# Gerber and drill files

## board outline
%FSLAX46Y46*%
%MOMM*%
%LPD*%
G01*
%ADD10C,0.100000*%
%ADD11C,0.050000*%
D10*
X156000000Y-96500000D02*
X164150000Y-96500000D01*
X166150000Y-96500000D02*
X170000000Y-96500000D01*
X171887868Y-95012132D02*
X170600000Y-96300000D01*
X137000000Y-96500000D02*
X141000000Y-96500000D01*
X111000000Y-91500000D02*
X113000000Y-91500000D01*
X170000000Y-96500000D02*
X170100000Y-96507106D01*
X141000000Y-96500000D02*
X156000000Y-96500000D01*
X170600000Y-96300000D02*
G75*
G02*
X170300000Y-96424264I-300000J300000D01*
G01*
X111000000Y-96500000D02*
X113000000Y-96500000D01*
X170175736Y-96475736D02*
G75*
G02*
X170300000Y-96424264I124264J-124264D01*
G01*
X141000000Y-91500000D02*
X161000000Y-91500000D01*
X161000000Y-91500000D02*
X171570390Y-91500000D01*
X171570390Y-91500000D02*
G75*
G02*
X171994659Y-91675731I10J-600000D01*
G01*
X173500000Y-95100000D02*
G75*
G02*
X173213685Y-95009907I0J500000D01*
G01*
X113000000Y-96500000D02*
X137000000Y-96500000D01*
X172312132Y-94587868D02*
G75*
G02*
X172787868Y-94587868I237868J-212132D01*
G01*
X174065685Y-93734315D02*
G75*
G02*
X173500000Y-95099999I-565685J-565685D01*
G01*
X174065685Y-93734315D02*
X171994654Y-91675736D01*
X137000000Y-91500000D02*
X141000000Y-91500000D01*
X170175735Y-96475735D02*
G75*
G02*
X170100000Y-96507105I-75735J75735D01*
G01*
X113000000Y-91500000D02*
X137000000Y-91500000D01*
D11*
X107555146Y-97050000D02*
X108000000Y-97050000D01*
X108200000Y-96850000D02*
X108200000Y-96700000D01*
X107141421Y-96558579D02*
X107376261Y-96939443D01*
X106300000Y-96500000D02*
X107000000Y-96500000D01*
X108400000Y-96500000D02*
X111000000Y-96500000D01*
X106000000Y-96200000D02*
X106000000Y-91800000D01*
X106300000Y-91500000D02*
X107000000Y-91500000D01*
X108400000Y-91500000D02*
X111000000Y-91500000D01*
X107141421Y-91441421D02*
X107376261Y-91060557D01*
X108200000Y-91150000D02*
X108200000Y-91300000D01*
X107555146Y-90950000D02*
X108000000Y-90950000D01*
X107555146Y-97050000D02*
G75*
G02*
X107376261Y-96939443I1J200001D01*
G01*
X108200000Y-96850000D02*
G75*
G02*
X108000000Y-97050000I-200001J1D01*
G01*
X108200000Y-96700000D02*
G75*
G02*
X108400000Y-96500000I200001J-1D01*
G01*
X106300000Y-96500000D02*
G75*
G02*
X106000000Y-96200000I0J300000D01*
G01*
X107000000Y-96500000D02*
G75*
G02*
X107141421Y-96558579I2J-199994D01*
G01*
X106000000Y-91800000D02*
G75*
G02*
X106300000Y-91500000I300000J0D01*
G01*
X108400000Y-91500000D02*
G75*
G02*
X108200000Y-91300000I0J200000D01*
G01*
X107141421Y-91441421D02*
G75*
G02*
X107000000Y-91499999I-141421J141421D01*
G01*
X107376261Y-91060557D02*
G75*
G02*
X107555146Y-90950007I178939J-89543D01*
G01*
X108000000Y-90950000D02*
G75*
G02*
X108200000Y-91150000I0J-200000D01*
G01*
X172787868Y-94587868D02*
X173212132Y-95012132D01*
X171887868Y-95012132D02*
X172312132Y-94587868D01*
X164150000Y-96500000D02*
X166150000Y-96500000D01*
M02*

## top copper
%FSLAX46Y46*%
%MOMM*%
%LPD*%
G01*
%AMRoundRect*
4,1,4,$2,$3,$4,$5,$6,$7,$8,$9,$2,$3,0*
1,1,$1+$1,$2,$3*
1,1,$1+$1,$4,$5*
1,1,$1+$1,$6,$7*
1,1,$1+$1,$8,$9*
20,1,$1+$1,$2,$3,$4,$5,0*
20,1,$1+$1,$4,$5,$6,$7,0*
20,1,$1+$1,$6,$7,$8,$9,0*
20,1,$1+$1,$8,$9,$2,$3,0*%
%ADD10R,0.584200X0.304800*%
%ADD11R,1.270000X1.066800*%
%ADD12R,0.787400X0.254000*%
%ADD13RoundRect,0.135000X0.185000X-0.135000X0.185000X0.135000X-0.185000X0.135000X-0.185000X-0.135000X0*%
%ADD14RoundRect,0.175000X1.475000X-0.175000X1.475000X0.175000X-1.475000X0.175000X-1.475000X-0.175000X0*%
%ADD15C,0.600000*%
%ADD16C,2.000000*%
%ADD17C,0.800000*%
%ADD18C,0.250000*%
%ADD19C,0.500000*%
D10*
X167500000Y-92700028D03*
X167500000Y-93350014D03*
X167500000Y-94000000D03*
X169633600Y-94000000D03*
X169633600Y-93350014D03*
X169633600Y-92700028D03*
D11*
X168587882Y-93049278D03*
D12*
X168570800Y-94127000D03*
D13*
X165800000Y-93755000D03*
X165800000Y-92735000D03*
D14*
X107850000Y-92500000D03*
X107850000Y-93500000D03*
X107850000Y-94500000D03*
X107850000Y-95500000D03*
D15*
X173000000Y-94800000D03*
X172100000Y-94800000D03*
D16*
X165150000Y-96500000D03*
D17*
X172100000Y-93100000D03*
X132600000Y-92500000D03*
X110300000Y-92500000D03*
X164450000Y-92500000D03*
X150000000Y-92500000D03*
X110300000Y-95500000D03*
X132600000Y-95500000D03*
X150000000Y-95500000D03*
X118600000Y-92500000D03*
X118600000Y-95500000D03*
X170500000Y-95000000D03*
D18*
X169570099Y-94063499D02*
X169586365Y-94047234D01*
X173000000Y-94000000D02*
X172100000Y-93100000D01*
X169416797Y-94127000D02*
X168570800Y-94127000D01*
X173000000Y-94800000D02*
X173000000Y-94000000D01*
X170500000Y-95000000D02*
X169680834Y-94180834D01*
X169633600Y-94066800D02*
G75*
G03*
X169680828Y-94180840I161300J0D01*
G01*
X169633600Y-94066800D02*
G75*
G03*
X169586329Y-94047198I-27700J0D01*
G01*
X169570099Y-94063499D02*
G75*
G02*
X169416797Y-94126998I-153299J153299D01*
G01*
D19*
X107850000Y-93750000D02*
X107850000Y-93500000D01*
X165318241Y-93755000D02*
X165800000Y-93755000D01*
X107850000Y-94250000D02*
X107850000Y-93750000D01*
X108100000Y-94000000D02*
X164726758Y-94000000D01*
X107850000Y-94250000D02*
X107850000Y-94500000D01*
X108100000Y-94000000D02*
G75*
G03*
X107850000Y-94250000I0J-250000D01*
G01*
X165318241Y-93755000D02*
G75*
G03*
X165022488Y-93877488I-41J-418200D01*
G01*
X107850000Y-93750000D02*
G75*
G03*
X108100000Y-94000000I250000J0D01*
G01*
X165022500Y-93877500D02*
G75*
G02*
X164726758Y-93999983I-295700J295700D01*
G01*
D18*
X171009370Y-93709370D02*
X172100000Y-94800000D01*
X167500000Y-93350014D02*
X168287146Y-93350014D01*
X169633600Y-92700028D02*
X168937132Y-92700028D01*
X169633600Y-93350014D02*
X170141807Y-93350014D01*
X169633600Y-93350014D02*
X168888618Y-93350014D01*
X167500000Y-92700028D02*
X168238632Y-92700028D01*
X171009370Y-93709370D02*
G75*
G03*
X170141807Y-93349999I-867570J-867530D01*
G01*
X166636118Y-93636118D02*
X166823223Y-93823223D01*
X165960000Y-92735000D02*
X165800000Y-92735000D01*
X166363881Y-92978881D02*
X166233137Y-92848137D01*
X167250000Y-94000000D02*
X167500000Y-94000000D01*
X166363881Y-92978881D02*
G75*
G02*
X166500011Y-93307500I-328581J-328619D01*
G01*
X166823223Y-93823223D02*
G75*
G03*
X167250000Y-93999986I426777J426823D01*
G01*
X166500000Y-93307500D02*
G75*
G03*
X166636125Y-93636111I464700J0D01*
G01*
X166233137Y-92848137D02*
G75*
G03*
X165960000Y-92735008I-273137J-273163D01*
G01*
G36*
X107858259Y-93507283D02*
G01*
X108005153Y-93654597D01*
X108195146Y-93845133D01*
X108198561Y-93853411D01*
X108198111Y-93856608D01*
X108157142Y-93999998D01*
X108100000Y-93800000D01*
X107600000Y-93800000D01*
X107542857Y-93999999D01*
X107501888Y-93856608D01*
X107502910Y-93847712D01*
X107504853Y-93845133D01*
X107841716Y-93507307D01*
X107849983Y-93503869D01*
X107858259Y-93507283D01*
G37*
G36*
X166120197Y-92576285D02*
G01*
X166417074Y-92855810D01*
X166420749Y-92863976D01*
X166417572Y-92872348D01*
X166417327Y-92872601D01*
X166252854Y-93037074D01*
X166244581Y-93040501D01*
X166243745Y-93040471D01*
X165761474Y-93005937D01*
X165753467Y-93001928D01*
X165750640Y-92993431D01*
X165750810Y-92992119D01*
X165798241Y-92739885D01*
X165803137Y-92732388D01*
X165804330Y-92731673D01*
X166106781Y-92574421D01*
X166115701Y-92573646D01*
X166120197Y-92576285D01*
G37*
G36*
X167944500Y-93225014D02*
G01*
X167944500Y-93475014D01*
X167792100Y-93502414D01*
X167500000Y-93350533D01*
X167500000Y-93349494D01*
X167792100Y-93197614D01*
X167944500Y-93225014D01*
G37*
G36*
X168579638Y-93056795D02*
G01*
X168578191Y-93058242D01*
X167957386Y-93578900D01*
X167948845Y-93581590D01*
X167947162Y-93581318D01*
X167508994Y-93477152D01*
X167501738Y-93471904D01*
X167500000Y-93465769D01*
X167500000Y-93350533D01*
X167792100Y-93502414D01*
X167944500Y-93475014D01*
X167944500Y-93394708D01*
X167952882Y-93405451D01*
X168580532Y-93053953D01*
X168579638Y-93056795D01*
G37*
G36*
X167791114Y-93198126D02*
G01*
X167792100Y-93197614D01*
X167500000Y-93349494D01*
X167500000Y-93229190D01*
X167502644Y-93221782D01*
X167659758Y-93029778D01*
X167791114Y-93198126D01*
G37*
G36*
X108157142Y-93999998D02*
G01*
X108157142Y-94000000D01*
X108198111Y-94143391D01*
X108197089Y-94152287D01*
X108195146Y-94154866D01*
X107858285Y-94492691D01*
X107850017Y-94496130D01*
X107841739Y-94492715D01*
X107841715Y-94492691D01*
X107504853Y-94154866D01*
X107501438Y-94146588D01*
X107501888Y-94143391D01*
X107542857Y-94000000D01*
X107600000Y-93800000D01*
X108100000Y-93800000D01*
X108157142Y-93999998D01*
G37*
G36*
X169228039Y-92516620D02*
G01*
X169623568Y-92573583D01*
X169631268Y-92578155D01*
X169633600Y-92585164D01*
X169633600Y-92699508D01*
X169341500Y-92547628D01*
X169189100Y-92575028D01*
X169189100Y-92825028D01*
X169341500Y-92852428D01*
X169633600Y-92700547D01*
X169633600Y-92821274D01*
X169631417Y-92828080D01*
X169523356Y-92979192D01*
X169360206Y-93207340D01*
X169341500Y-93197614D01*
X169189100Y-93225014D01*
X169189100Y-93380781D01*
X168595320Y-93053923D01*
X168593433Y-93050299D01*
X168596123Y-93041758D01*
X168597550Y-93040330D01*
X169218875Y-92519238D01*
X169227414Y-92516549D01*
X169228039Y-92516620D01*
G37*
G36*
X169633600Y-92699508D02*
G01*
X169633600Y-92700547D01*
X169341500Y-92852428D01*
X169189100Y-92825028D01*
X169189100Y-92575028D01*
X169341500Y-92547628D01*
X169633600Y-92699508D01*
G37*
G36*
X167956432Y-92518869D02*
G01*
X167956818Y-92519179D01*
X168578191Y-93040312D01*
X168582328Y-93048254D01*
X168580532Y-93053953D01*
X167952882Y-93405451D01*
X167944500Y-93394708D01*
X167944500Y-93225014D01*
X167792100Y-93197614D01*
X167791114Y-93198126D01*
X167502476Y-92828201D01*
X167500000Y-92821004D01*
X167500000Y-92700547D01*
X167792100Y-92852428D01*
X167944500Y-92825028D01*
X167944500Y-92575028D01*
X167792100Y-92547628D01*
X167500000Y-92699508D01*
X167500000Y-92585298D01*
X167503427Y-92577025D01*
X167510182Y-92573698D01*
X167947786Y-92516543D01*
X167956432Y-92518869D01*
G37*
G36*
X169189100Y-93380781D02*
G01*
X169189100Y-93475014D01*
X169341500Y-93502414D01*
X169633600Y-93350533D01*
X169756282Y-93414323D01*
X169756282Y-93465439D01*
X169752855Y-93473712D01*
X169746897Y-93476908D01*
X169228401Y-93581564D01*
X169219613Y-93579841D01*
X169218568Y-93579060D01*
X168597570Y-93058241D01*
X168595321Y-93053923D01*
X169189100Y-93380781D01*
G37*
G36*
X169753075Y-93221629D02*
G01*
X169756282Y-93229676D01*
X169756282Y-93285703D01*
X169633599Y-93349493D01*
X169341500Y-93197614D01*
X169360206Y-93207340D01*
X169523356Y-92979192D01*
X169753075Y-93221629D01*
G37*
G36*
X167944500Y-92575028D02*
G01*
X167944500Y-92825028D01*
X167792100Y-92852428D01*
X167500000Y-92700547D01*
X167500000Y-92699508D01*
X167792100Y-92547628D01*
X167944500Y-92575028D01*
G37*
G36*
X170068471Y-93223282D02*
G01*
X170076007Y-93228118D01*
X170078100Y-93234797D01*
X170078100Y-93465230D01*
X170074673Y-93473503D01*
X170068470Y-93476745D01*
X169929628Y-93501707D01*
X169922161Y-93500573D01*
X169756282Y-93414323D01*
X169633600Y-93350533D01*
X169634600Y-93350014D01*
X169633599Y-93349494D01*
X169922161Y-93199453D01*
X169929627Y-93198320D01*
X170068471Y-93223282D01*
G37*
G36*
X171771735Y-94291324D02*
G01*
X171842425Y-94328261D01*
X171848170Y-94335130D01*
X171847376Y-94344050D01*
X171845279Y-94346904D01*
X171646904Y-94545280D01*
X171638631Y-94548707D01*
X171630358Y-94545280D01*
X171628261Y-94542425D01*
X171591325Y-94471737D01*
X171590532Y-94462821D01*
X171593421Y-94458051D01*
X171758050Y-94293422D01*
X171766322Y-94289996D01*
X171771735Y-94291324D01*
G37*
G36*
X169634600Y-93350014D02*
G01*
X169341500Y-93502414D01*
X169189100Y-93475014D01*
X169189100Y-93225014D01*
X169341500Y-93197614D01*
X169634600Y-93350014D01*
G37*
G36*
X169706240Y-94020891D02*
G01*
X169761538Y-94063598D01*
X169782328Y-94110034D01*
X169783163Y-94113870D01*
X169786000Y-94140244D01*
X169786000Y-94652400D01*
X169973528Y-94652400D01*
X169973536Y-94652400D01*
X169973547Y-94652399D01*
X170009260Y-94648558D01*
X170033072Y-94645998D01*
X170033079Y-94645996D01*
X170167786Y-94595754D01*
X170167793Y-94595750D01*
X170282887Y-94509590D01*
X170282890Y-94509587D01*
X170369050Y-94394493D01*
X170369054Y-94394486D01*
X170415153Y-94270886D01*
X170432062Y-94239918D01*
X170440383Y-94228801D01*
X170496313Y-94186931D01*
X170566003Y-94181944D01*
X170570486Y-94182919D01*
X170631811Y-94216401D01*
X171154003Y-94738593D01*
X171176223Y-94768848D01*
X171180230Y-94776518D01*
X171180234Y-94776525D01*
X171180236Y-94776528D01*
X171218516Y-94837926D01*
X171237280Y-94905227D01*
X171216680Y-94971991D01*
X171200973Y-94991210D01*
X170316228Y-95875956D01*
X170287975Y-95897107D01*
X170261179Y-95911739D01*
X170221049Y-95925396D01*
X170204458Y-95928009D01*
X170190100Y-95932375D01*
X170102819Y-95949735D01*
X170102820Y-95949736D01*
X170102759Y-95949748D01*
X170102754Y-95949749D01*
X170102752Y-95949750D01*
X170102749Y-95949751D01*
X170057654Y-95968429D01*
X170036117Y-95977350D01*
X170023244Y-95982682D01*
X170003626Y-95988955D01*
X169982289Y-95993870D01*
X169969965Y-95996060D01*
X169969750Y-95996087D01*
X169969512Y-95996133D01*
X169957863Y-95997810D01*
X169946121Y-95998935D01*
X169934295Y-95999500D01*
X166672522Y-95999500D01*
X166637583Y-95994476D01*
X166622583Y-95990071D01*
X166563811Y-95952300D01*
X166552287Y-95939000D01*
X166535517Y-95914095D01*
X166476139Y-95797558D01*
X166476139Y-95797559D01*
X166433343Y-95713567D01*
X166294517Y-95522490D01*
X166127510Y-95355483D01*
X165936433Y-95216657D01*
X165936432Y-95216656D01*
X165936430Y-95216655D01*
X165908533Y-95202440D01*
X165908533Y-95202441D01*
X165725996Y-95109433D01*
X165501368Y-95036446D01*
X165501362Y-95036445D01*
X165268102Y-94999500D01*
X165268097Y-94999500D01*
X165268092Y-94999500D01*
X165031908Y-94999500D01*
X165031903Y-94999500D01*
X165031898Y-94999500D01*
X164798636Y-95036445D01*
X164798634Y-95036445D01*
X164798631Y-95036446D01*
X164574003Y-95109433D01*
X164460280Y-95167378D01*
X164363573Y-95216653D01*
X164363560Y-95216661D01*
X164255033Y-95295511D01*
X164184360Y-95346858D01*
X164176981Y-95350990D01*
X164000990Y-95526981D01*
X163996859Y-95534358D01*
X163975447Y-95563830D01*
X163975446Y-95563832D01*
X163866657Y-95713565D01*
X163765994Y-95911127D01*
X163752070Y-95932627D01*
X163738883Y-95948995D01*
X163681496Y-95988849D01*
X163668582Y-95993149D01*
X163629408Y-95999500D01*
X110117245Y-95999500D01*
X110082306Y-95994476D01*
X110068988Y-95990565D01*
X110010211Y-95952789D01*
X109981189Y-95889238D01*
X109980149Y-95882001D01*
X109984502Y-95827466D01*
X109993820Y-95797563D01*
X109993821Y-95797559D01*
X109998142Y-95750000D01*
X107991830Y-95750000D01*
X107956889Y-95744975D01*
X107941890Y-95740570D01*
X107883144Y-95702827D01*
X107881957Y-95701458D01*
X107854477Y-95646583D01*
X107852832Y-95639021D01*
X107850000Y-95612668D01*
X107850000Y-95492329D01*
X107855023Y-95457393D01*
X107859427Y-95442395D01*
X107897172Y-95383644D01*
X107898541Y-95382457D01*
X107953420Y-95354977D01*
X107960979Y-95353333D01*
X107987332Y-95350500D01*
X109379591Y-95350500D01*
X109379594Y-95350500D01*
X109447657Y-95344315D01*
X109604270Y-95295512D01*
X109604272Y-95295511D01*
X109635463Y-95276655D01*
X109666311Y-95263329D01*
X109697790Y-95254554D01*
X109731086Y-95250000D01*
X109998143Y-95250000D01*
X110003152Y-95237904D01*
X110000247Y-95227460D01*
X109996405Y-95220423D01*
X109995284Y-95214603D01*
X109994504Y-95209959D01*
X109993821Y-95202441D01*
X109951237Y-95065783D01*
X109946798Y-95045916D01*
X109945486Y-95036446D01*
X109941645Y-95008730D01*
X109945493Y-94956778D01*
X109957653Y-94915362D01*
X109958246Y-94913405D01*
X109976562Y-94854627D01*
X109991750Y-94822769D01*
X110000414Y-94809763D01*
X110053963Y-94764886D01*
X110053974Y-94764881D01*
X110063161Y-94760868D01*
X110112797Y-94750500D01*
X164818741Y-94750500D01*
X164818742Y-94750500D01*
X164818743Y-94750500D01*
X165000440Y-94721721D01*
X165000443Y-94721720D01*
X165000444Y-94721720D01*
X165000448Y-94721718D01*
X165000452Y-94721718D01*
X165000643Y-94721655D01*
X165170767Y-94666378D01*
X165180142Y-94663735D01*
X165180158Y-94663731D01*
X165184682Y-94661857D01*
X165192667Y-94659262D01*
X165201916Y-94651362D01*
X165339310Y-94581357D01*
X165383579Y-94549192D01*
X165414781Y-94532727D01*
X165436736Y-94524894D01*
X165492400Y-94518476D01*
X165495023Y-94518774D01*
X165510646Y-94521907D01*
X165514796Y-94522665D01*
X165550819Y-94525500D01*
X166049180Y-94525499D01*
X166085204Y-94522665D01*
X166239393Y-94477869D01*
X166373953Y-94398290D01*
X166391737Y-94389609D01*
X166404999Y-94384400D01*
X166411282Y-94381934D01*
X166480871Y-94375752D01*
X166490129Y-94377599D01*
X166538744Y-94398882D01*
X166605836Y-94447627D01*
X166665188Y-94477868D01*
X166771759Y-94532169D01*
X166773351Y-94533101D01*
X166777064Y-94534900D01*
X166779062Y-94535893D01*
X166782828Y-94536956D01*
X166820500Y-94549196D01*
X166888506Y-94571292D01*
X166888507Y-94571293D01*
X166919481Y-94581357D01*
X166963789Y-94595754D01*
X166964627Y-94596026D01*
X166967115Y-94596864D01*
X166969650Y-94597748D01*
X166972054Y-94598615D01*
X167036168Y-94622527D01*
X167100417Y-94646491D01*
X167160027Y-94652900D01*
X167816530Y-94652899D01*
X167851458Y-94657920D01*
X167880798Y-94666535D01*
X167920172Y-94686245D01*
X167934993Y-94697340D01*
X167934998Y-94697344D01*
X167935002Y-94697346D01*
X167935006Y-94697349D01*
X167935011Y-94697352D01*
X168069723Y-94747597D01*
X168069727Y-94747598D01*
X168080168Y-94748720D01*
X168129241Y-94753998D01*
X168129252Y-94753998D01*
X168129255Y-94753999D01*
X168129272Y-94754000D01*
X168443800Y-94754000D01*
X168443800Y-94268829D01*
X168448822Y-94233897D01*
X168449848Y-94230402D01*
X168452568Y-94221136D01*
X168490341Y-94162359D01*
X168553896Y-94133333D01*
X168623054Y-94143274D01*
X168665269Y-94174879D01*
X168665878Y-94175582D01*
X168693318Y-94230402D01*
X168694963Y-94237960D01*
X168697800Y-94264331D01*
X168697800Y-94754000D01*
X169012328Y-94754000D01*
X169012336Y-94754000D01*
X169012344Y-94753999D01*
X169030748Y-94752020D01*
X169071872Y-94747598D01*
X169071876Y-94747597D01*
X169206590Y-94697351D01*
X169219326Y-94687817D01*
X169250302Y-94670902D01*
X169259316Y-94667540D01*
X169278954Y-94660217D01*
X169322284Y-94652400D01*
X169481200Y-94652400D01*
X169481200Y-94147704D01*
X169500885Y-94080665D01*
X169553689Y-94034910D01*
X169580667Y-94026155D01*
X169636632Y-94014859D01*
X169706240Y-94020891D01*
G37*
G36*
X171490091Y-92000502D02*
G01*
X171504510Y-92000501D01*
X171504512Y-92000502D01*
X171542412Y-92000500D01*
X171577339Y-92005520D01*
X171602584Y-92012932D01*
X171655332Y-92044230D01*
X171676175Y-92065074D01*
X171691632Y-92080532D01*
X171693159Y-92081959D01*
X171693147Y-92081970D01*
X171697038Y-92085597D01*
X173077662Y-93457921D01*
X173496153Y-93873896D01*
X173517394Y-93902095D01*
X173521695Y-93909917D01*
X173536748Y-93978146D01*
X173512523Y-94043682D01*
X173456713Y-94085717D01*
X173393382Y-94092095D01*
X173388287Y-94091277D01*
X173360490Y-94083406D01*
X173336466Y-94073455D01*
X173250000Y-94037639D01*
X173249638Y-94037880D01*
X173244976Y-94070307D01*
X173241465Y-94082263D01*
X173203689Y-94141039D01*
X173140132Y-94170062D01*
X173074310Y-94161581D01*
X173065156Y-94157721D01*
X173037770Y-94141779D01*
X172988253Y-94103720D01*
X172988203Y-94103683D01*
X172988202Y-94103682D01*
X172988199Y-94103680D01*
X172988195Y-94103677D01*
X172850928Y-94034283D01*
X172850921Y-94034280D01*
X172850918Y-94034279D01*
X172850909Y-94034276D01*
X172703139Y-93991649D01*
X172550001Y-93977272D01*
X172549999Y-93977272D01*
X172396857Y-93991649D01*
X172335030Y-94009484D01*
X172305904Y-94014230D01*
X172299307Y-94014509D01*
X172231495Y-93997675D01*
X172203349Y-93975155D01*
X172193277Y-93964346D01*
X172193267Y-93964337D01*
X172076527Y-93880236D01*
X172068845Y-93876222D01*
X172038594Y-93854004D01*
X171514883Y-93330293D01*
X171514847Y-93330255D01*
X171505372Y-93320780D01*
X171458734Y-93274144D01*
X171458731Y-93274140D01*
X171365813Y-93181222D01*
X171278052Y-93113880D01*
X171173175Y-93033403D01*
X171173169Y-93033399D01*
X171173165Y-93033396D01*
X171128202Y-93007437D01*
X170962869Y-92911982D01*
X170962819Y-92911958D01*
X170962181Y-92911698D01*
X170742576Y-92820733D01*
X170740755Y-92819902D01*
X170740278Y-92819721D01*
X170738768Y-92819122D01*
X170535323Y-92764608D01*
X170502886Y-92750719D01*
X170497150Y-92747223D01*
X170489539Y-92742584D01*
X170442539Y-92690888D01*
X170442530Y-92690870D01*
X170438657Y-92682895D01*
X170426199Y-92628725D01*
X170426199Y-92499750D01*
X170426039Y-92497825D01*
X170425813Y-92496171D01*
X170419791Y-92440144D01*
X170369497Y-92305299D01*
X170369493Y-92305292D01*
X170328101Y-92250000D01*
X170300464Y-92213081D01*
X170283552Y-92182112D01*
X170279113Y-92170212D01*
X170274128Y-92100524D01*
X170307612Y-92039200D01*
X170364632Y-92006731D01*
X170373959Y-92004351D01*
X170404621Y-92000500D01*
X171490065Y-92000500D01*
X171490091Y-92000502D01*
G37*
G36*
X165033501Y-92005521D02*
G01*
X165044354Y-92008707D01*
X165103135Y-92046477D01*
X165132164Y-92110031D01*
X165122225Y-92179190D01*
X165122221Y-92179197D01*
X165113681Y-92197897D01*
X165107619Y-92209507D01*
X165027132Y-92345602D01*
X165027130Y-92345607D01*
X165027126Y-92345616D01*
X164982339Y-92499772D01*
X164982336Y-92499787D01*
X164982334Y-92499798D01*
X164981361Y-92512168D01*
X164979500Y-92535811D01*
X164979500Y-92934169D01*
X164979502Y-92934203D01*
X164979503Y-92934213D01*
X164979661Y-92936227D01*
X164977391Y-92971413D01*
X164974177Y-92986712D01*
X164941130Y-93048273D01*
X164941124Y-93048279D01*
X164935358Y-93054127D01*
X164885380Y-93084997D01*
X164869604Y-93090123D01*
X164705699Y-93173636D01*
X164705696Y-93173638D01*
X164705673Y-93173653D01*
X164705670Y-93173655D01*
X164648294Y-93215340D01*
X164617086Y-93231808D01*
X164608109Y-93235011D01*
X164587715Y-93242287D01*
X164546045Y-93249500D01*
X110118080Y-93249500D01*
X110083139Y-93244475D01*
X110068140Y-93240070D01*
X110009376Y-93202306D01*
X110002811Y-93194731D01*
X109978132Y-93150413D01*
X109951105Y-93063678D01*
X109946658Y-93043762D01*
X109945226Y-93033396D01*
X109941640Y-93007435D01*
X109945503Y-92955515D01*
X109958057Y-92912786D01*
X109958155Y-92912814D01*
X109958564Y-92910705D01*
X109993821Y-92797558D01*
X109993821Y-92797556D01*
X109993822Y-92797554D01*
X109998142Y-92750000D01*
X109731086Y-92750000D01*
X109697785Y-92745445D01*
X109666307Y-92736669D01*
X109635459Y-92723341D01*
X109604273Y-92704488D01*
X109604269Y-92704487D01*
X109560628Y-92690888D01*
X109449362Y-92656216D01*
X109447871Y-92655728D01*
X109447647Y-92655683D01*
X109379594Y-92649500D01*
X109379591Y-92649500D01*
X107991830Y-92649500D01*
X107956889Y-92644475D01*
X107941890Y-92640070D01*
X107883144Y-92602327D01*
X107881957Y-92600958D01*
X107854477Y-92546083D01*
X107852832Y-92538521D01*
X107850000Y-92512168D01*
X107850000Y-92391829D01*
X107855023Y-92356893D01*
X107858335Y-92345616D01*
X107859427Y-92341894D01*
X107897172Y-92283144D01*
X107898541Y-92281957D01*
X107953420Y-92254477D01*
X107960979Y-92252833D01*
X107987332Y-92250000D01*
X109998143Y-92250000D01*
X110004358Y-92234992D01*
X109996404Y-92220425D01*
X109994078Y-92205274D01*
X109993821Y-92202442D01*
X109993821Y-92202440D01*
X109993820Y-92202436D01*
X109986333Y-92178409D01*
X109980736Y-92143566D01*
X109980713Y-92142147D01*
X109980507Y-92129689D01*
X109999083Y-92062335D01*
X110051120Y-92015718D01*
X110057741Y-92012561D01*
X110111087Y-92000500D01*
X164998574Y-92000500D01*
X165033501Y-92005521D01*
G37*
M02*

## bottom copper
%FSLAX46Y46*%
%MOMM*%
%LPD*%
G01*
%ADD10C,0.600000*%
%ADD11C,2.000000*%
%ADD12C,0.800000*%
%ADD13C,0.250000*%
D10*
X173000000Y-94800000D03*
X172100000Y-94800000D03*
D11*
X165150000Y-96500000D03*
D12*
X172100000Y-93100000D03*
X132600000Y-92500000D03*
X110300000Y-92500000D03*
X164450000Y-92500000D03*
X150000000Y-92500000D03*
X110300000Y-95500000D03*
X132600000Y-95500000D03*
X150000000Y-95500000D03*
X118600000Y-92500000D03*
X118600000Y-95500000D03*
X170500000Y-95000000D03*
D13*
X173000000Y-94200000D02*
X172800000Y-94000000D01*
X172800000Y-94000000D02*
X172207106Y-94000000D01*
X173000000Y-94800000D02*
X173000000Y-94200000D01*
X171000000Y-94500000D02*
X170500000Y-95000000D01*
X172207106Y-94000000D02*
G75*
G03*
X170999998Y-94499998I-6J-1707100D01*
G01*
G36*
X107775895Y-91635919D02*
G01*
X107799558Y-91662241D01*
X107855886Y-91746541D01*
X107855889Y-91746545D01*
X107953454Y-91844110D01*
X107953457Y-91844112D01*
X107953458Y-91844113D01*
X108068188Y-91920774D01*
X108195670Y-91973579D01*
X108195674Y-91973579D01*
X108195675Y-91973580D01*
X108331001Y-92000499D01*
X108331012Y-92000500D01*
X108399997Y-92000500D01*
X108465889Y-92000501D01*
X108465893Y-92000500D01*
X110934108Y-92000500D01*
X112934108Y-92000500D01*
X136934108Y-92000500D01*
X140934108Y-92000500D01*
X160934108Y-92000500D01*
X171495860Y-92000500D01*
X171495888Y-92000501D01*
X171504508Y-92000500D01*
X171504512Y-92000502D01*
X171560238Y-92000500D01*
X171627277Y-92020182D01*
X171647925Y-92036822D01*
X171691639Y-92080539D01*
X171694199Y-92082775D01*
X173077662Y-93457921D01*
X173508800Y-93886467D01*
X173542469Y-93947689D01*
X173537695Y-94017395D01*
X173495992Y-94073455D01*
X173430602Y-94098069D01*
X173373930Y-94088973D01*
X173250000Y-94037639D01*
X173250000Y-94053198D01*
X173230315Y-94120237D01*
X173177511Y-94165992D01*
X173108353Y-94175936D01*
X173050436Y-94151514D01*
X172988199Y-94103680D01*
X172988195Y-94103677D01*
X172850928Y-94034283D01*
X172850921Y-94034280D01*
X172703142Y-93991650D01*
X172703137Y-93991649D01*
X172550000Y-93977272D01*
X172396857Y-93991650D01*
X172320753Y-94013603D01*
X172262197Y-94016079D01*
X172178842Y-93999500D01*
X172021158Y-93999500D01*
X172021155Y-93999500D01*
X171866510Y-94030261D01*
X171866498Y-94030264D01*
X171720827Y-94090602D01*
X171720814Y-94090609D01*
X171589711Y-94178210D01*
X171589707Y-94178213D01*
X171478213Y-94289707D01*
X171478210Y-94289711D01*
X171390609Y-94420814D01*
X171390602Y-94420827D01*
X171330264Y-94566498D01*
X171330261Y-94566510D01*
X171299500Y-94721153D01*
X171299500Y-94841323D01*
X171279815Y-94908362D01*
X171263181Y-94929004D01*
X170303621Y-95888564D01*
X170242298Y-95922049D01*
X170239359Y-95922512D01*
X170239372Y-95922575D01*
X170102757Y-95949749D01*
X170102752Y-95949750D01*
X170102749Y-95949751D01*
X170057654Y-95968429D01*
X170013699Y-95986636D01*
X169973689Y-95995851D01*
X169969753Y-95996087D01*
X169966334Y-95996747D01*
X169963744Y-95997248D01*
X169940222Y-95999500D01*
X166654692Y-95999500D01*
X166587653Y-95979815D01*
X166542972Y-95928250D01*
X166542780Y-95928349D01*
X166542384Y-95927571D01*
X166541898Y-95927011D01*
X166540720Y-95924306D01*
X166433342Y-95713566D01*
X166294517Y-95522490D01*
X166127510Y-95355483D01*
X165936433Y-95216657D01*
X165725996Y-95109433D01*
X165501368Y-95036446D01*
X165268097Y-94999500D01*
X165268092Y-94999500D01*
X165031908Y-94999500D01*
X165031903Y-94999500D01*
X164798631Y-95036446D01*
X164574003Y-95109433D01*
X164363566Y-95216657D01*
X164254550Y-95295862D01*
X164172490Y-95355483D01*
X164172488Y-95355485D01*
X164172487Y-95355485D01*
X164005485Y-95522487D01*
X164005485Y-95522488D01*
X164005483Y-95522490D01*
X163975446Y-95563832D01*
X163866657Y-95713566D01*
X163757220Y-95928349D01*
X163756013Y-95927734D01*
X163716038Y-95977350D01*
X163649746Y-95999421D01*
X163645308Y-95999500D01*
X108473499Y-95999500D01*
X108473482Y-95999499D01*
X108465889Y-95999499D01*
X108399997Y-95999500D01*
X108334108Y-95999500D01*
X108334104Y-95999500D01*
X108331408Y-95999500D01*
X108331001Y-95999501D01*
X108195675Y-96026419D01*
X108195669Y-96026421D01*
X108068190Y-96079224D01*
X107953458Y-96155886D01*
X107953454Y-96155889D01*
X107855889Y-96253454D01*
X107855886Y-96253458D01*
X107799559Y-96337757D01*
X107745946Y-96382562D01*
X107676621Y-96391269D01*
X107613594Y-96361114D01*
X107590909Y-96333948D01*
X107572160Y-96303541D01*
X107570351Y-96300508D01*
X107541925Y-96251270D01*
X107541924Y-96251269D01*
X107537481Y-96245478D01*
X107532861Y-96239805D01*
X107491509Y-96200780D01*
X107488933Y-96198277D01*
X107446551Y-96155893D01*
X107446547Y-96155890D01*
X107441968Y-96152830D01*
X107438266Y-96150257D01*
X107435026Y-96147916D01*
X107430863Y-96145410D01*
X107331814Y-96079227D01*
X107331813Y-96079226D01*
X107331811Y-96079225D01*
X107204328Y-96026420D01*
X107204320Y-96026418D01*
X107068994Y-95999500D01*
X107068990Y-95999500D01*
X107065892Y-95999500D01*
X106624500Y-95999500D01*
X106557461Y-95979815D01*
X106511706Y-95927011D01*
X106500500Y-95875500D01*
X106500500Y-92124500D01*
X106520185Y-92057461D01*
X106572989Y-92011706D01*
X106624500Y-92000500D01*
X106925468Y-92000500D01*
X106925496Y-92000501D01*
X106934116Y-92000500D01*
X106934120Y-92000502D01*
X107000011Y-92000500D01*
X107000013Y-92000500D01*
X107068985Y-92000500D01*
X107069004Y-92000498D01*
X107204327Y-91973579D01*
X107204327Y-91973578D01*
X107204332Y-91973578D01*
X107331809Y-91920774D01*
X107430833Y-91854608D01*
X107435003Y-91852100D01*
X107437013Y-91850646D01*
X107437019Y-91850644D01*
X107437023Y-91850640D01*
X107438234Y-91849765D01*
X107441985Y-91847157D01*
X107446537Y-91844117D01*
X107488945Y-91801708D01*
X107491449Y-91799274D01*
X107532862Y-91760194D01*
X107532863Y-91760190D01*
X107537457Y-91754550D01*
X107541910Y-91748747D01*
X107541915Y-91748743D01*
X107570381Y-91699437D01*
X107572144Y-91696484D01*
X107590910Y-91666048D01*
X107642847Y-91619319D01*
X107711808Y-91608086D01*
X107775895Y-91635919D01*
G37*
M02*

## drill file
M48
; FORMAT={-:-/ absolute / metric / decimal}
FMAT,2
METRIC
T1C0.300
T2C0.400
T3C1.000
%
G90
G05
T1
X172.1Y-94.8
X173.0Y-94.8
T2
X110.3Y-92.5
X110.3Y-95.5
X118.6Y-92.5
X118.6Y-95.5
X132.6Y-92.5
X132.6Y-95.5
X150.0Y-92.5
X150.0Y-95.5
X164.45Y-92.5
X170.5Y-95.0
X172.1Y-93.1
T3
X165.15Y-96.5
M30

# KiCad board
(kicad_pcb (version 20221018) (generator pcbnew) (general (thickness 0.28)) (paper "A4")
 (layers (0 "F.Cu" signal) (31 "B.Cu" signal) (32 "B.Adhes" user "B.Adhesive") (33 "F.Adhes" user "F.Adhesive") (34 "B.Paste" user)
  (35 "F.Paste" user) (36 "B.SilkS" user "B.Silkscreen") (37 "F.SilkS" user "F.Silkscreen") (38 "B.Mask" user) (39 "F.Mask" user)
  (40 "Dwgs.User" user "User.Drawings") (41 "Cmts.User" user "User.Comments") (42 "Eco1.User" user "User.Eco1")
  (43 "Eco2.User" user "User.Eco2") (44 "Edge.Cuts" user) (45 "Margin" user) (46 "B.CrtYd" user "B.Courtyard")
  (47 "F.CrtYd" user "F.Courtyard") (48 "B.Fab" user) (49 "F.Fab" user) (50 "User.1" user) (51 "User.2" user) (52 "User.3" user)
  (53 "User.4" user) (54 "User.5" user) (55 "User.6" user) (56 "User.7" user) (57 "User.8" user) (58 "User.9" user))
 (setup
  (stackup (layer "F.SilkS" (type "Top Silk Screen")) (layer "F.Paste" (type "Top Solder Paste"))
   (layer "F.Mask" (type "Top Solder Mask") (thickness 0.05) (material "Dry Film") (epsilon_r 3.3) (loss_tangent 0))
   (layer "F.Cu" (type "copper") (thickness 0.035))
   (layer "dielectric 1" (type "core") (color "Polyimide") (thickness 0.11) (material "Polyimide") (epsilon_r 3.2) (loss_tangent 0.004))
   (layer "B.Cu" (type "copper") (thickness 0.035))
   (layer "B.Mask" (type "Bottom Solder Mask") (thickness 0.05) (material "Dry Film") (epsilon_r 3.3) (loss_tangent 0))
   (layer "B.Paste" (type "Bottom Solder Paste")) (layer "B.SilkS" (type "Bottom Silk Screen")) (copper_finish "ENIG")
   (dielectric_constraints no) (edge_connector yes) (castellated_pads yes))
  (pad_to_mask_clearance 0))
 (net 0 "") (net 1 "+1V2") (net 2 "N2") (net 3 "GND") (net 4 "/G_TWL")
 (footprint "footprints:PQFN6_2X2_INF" (layer "F.Cu") (at 168.5668 93.350014)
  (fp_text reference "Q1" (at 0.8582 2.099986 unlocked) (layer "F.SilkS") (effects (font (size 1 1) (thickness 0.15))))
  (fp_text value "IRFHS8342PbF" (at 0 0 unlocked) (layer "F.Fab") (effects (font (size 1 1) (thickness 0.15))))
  (pad "1" smd rect (at -1.0668 -0.649986) (size 0.5842 0.3048) (layers "F.Cu" "F.Paste" "F.Mask") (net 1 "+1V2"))
  (pad "2" smd rect (at -1.0668 0) (size 0.5842 0.3048) (layers "F.Cu" "F.Paste" "F.Mask") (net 1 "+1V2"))
  (pad "3" smd rect (at -1.0668 0.649986) (size 0.5842 0.3048) (layers "F.Cu" "F.Paste" "F.Mask") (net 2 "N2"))
  (pad "4" smd rect (at 1.0668 0.649986) (size 0.5842 0.3048) (layers "F.Cu" "F.Paste" "F.Mask") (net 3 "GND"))
  (pad "5" smd rect (at 1.0668 0) (size 0.5842 0.3048) (layers "F.Cu" "F.Paste" "F.Mask") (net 1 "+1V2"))
  (pad "6" smd rect (at 1.0668 -0.649986) (size 0.5842 0.3048) (layers "F.Cu" "F.Paste" "F.Mask") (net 1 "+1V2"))
  (pad "7" smd rect (at 0.021082 -0.300736) (size 1.27 1.0668) (layers "F.Cu" "F.Paste" "F.Mask") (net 1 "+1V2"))
  (pad "8" smd rect (at 0.004 0.776986) (size 0.7874 0.254) (layers "F.Cu" "F.Paste" "F.Mask") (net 3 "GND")))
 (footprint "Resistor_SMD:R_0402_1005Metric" (layer "F.Cu") (at 165.8 93.245 90)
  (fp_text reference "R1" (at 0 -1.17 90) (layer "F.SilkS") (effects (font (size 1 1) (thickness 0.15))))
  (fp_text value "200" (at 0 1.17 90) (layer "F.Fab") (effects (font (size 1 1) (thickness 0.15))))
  (pad "1" smd roundrect (at -0.51 0 90) (size 0.54 0.64) (layers "F.Cu" "F.Paste" "F.Mask") (roundrect_rratio 0.25) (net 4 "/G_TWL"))
  (pad "2" smd roundrect (at 0.51 0 90) (size 0.54 0.64) (layers "F.Cu" "F.Paste" "F.Mask") (roundrect_rratio 0.25) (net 2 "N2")))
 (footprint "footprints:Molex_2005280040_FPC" (layer "F.Cu") (at 111 94 90)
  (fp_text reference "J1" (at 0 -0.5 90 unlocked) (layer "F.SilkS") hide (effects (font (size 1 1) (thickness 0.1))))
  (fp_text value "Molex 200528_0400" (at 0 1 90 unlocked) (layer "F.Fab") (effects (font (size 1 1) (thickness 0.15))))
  (fp_line (start -3.05 -3.444854) (end -3.05 -3) (stroke (width 0.05) (type default)) (layer "Edge.Cuts"))
  (fp_line (start -2.85 -2.8) (end -2.7 -2.8) (stroke (width 0.05) (type default)) (layer "Edge.Cuts"))
  (fp_line (start -2.558579 -3.858579) (end -2.939443 -3.623739) (stroke (width 0.05) (type default)) (layer "Edge.Cuts"))
  (fp_line (start -2.5 -4.7) (end -2.5 -4) (stroke (width 0.05) (type default)) (layer "Edge.Cuts"))
  (fp_line (start -2.5 -2.6) (end -2.5 0) (stroke (width 0.05) (type default)) (layer "Edge.Cuts"))
  (fp_line (start -2.2 -5) (end 2.2 -5) (stroke (width 0.05) (type default)) (layer "Edge.Cuts"))
  (fp_line (start 2.5 -4.7) (end 2.5 -4) (stroke (width 0.05) (type default)) (layer "Edge.Cuts"))
  (fp_line (start 2.5 -2.6) (end 2.5 0) (stroke (width 0.05) (type default)) (layer "Edge.Cuts"))
  (fp_line (start 2.558579 -3.858579) (end 2.939443 -3.623739) (stroke (width 0.05) (type default)) (layer "Edge.Cuts"))
  (fp_line (start 2.85 -2.8) (end 2.7 -2.8) (stroke (width 0.05) (type default)) (layer "Edge.Cuts"))
  (fp_line (start 3.05 -3.444854) (end 3.05 -3) (stroke (width 0.05) (type default)) (layer "Edge.Cuts"))
  (fp_arc (start -3.05 -3.444854) (mid -3.02013 -3.55) (end -2.939443 -3.623739) (stroke (width 0.05) (type default)) (layer "Edge.Cuts"))
  (fp_arc (start -2.85 -2.8) (mid -2.991421 -2.858579) (end -3.05 -3) (stroke (width 0.05) (type default)) (layer "Edge.Cuts"))
  (fp_arc (start -2.7 -2.8) (mid -2.558579 -2.741421) (end -2.5 -2.6) (stroke (width 0.05) (type default)) (layer "Edge.Cuts"))
  (fp_arc (start -2.5 -4.7) (mid -2.412132 -4.912132) (end -2.2 -5) (stroke (width 0.05) (type default)) (layer "Edge.Cuts"))
  (fp_arc (start -2.5 -4) (mid -2.515224 -3.923463) (end -2.558579 -3.858579) (stroke (width 0.05) (type default)) (layer "Edge.Cuts"))
  (fp_arc (start 2.2 -5) (mid 2.412132 -4.912132) (end 2.5 -4.7) (stroke (width 0.05) (type default)) (layer "Edge.Cuts"))
  (fp_arc (start 2.5 -2.6) (mid 2.558579 -2.741421) (end 2.7 -2.8) (stroke (width 0.05) (type default)) (layer "Edge.Cuts"))
  (fp_arc (start 2.558579 -3.858579) (mid 2.515225 -3.923464) (end 2.5 -4) (stroke (width 0.05) (type default)) (layer "Edge.Cuts"))
  (fp_arc (start 2.939443 -3.623739) (mid 3.020112 -3.54999) (end 3.05 -3.444854) (stroke (width 0.05) (type default)) (layer "Edge.Cuts"))
  (fp_arc (start 3.05 -3) (mid 2.991421 -2.858579) (end 2.85 -2.8) (stroke (width 0.05) (type default)) (layer "Edge.Cuts"))
  (pad "1" smd roundrect (at 1.5 -3.15 90) (size 0.7 3.3) (layers "F.Cu" "F.Mask") (roundrect_rratio 0.25) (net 3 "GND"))
  (pad "2" smd roundrect (at 0.5 -3.15 90) (size 0.7 3.3) (layers "F.Cu" "F.Mask") (roundrect_rratio 0.25) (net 4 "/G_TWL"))
  (pad "3" smd roundrect (at -0.5 -3.15 90) (size 0.7 3.3) (layers "F.Cu" "F.Mask") (roundrect_rratio 0.25) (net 4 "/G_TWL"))
  (pad "4" smd roundrect (at -1.5 -3.15 90) (size 0.7 3.3) (layers "F.Cu" "F.Mask") (roundrect_rratio 0.25) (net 3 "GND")))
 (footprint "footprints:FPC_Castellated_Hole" (layer "F.Cu") (at 173 94.8 -45)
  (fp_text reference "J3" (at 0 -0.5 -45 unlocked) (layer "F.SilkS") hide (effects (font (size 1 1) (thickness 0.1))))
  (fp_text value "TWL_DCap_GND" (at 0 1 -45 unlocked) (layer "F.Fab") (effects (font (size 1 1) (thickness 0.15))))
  (fp_line (start -0.3 0) (end 0.3 0) (stroke (width 0.05) (type default)) (layer "Edge.Cuts"))
  (pad "1" thru_hole circle (at 0 0 315) (size 0.6 0.6) (drill 0.3) (layers "*.Cu" "*.Mask") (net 3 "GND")))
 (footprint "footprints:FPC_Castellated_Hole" (layer "F.Cu") (at 172.1 94.8 45)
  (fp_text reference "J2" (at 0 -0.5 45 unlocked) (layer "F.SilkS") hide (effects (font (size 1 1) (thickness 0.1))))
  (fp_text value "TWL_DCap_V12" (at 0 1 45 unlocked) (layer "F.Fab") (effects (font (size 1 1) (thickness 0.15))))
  (fp_line (start -0.3 0) (end 0.3 0) (stroke (width 0.05) (type default)) (layer "Edge.Cuts"))
  (pad "1" thru_hole circle (at 0 0 45) (size 0.6 0.6) (drill 0.3) (layers "*.Cu" "*.Mask") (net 1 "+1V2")))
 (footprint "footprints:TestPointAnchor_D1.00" (layer "F.Cu") (at 165.15 96.5)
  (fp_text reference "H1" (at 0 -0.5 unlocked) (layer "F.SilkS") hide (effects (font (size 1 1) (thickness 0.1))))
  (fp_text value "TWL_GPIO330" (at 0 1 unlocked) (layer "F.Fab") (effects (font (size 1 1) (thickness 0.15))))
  (fp_line (start -1 0) (end 1 0) (stroke (width 0.05) (type default)) (layer "Edge.Cuts"))
  (pad "1" thru_hole circle (at 0 0) (size 2 2) (drill 1) (layers "*.Cu" "*.Mask")))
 (gr_line (start 156 96.5) (end 164.15 96.5) (stroke (width 0.1) (type default)) (layer "Edge.Cuts"))
 (gr_line (start 166.15 96.5) (end 170 96.5) (stroke (width 0.1) (type default)) (layer "Edge.Cuts"))
 (gr_line (start 171.887868 95.012132) (end 170.6 96.3) (stroke (width 0.1) (type default)) (layer "Edge.Cuts"))
 (gr_line (start 137 96.5) (end 141 96.5) (stroke (width 0.1) (type default)) (layer "Edge.Cuts"))
 (gr_line (start 111 91.5) (end 113 91.5) (stroke (width 0.1) (type default)) (layer "Edge.Cuts"))
 (gr_line (start 170 96.5) (end 170.1 96.507106) (stroke (width 0.1) (type default)) (layer "Edge.Cuts"))
 (gr_line (start 141 96.5) (end 156 96.5) (stroke (width 0.1) (type default)) (layer "Edge.Cuts"))
 (gr_arc (start 170.6 96.3) (mid 170.462359 96.391969) (end 170.3 96.424264) (stroke (width 0.1) (type default)) (layer "Edge.Cuts"))
 (gr_line (start 111 96.5) (end 113 96.5) (stroke (width 0.1) (type default)) (layer "Edge.Cuts"))
 (gr_arc (start 170.175736 96.475736) (mid 170.232749 96.437641) (end 170.3 96.424264) (stroke (width 0.1) (type default))
  (layer "Edge.Cuts"))
 (gr_line (start 141 91.5) (end 161 91.5) (stroke (width 0.1) (type default)) (layer "Edge.Cuts"))
 (gr_line (start 161 91.5) (end 171.57039 91.5) (stroke (width 0.1) (type default)) (layer "Edge.Cuts"))
 (gr_arc (start 171.57039 91.5) (mid 171.800001 91.545669) (end 171.994654 91.675736) (stroke (width 0.1) (type default))
  (layer "Edge.Cuts"))
 (gr_arc (start 173.5 95.1) (mid 173.349923 95.076945) (end 173.213685 95.009907) (stroke (width 0.1) (type default)) (layer "Edge.Cuts"))
 (gr_line (start 113 96.5) (end 137 96.5) (stroke (width 0.1) (type default)) (layer "Edge.Cuts"))
 (gr_arc (start 172.312132 94.587868) (mid 172.55 94.481282) (end 172.787868 94.587868) (stroke (width 0.1) (type default))
  (layer "Edge.Cuts"))
 (gr_arc (start 174.065685 93.734315) (mid 174.239103 94.606147) (end 173.5 95.1) (stroke (width 0.1) (type default)) (layer "Edge.Cuts"))
 (gr_line (start 174.065685 93.734315) (end 171.994654 91.675736) (stroke (width 0.1) (type default)) (layer "Edge.Cuts"))
 (gr_line (start 137 91.5) (end 141 91.5) (stroke (width 0.1) (type default)) (layer "Edge.Cuts"))
 (gr_arc (start 170.175735 96.475735) (mid 170.140988 96.498953) (end 170.1 96.507106) (stroke (width 0.1) (type default))
  (layer "Edge.Cuts"))
 (gr_line (start 113 91.5) (end 137 91.5) (stroke (width 0.1) (type default)) (layer "Edge.Cuts"))
 (segment (start 169.570099 94.063499) (end 169.586365 94.047234) (width 0.25) (layer "F.Cu") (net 3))
 (segment (start 173 94) (end 172.1 93.1) (width 0.25) (layer "F.Cu") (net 3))
 (segment (start 169.416797 94.127) (end 168.5708 94.127) (width 0.25) (layer "F.Cu") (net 3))
 (segment (start 173 94.8) (end 173 94) (width 0.25) (layer "F.Cu") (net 3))
 (segment (start 170.5 95) (end 169.680834 94.180834) (width 0.25) (layer "F.Cu") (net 3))
 (via (at 172.1 93.1) (size 0.8) (drill 0.4) (layers "F.Cu" "B.Cu") (free) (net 3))
 (via (at 132.6 92.5) (size 0.8) (drill 0.4) (layers "F.Cu" "B.Cu") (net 3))
 (via (at 110.3 92.5) (size 0.8) (drill 0.4) (layers "F.Cu" "B.Cu") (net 3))
 (via (at 164.45 92.5) (size 0.8) (drill 0.4) (layers "F.Cu" "B.Cu") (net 3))
 (via (at 150 92.5) (size 0.8) (drill 0.4) (layers "F.Cu" "B.Cu") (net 3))
 (via (at 110.3 95.5) (size 0.8) (drill 0.4) (layers "F.Cu" "B.Cu") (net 3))
 (via (at 132.6 95.5) (size 0.8) (drill 0.4) (layers "F.Cu" "B.Cu") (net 3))
 (via (at 150 95.5) (size 0.8) (drill 0.4) (layers "F.Cu" "B.Cu") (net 3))
 (via (at 118.6 92.5) (size 0.8) (drill 0.4) (layers "F.Cu" "B.Cu") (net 3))
 (via (at 118.6 95.5) (size 0.8) (drill 0.4) (layers "F.Cu" "B.Cu") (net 3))
 (via (at 170.5 95) (size 0.8) (drill 0.4) (layers "F.Cu" "B.Cu") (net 3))
 (arc (start 169.6336 94.0668) (mid 169.645875 94.128514) (end 169.680834 94.180834) (width 0.25) (layer "F.Cu") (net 3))
 (arc (start 169.6336 94.0668) (mid 169.616519 94.041236) (end 169.586365 94.047234) (width 0.25) (layer "F.Cu") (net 3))
 (arc (start 169.570099 94.063499) (mid 169.499763 94.110496) (end 169.416797 94.127) (width 0.25) (layer "F.Cu") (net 3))
 (segment (start 173 94.2) (end 172.8 94) (width 0.25) (layer "B.Cu") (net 3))
 (segment (start 172.8 94) (end 172.207106 94) (width 0.25) (layer "B.Cu") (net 3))
 (segment (start 173 94.8) (end 173 94.2) (width 0.25) (layer "B.Cu") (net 3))
 (segment (start 171 94.5) (end 170.5 95) (width 0.25) (layer "B.Cu") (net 3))
 (arc (start 172.207106 94) (mid 171.553825 94.129945) (end 171 94.5) (width 0.25) (layer "B.Cu") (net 3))
 (segment (start 107.85 93.75) (end 107.85 93.5) (width 0.5) (layer "F.Cu") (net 4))
 (segment (start 165.318241 93.755) (end 165.8 93.755) (width 0.5) (layer "F.Cu") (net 4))
 (segment (start 107.85 94.25) (end 107.85 93.75) (width 0.5) (layer "F.Cu") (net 4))
 (segment (start 108.1 94) (end 164.726758 94) (width 0.5) (layer "F.Cu") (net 4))
 (segment (start 107.85 94.25) (end 107.85 94.5) (width 0.5) (layer "F.Cu") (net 4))
 (arc (start 108.1 94) (mid 107.923223 94.073223) (end 107.85 94.25) (width 0.5) (layer "F.Cu") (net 4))
 (arc (start 165.318241 93.755) (mid 165.158187 93.786836) (end 165.0225 93.8775) (width 0.5) (layer "F.Cu") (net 4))
 (arc (start 107.85 93.75) (mid 107.923223 93.926776) (end 108.1 94) (width 0.5) (layer "F.Cu") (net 4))
 (arc (start 165.0225 93.8775) (mid 164.886812 93.968163) (end 164.726758 94) (width 0.5) (layer "F.Cu") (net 4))
 (segment (start 171.00937 93.70937) (end 172.1 94.8) (width 0.25) (layer "F.Cu") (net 1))
 (segment (start 167.5 93.350014) (end 168.287146 93.350014) (width 0.25) (layer "F.Cu") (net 1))
 (segment (start 169.6336 92.700028) (end 168.937132 92.700028) (width 0.25) (layer "F.Cu") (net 1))
 (segment (start 169.6336 93.350014) (end 170.141807 93.350014) (width 0.25) (layer "F.Cu") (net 1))
 (segment (start 169.6336 93.350014) (end 168.888618 93.350014) (width 0.25) (layer "F.Cu") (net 1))
 (segment (start 167.5 92.700028) (end 168.238632 92.700028) (width 0.25) (layer "F.Cu") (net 1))
 (arc (start 171.00937 93.70937) (mid 170.611328 93.443407) (end 170.141807 93.350014) (width 0.25) (layer "F.Cu") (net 1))
 (segment (start 166.636118 93.636118) (end 166.823223 93.823223) (width 0.25) (layer "F.Cu") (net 2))
 (segment (start 165.96 92.735) (end 165.8 92.735) (width 0.25) (layer "F.Cu") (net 2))
 (segment (start 166.363881 92.978881) (end 166.233137 92.848137) (width 0.25) (layer "F.Cu") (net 2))
 (segment (start 167.25 94) (end 167.5 94) (width 0.25) (layer "F.Cu") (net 2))
 (arc (start 166.363881 92.978881) (mid 166.464623 93.129652) (end 166.5 93.3075) (width 0.25) (layer "F.Cu") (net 2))
 (arc (start 166.823223 93.823223) (mid 167.01903 93.954057) (end 167.25 94) (width 0.25) (layer "F.Cu") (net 2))
 (arc (start 166.5 93.3075) (mid 166.535375 93.485346) (end 166.636118 93.636118) (width 0.25) (layer "F.Cu") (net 2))
 (arc (start 166.233137 92.848137) (mid 166.10782 92.764403) (end 165.96 92.735) (width 0.25) (layer "F.Cu") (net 2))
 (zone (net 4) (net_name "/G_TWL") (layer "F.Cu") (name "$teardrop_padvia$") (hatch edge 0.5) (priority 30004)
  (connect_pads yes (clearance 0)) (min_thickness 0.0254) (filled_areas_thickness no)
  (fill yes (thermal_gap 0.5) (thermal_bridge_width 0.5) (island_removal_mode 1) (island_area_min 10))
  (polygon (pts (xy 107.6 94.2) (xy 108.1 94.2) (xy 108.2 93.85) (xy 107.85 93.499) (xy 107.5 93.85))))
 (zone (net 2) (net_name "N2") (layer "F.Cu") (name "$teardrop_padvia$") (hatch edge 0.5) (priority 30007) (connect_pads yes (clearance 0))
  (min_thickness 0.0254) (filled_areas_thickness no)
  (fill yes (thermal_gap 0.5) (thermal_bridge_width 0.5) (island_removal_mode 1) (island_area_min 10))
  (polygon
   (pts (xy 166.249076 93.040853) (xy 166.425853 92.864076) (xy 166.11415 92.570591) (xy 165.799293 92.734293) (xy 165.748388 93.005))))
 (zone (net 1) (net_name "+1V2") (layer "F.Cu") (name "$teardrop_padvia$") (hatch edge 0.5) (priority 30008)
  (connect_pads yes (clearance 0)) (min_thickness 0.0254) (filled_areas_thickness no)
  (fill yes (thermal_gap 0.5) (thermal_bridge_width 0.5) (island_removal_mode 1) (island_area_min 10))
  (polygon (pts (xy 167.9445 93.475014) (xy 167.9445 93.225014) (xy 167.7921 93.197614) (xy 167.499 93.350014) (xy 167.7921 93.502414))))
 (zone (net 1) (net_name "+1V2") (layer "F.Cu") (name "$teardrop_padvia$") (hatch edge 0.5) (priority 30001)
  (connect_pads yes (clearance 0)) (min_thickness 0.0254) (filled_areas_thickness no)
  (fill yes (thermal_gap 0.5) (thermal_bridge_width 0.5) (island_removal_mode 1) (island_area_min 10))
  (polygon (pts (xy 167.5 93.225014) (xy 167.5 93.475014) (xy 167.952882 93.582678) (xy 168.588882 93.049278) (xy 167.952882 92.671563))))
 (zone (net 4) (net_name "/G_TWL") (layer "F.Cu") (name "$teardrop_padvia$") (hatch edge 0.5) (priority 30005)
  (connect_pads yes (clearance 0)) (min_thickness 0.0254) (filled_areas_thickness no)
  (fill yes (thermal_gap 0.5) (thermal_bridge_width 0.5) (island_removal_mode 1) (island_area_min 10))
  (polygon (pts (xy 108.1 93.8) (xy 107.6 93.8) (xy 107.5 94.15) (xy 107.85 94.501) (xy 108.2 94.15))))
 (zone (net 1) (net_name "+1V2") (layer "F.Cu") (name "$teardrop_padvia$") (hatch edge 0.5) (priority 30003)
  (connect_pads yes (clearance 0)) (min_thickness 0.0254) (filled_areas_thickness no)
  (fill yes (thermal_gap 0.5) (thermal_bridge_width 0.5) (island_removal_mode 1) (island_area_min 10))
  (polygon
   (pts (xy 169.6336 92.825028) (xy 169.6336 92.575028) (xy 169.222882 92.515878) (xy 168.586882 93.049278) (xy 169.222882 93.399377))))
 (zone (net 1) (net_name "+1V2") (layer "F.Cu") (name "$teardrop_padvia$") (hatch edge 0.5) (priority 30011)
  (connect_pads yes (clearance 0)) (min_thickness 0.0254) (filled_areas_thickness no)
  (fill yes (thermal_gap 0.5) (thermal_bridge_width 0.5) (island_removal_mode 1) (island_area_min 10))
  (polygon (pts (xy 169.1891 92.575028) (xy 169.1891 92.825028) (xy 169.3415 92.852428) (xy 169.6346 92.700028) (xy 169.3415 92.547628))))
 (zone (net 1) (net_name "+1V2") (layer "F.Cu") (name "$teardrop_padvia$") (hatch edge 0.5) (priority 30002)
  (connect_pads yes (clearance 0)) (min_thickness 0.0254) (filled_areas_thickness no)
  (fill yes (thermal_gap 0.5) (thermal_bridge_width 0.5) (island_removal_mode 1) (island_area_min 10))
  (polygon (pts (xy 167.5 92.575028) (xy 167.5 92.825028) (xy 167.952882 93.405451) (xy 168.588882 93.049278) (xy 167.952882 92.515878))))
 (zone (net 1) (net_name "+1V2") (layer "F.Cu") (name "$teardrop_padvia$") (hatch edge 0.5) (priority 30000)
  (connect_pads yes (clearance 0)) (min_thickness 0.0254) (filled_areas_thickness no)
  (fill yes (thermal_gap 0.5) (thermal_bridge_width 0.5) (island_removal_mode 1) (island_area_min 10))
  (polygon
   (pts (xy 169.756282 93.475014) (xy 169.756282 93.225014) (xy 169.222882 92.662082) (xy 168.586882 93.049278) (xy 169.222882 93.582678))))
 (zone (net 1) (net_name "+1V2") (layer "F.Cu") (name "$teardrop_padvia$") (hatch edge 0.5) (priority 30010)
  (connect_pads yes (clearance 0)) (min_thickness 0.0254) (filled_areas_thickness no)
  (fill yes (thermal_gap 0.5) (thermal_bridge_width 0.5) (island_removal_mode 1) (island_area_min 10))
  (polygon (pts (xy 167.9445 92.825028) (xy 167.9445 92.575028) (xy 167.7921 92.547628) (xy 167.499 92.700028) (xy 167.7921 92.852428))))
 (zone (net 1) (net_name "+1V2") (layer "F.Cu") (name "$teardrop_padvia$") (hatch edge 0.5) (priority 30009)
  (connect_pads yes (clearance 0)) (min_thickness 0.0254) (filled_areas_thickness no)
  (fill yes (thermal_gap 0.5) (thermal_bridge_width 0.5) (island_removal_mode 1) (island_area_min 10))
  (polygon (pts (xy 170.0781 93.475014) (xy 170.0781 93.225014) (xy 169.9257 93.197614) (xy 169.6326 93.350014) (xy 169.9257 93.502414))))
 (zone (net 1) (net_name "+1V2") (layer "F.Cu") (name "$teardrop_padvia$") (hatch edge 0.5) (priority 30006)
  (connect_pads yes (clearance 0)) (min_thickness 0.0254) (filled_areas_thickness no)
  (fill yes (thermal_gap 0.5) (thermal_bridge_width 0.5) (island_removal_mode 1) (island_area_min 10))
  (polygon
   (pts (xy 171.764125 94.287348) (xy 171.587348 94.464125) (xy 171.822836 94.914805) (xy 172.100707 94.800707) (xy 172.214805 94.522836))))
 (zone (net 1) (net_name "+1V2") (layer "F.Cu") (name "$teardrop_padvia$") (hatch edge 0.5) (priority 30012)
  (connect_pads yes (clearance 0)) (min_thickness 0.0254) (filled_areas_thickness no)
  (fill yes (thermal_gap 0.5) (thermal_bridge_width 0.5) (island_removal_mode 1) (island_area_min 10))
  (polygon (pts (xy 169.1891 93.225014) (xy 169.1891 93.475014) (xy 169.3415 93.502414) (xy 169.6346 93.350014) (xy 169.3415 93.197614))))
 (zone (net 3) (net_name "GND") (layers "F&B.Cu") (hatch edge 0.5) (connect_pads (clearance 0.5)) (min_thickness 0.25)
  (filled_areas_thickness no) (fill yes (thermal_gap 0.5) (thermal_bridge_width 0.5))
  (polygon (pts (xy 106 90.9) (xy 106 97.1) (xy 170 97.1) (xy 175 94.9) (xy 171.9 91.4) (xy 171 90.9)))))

